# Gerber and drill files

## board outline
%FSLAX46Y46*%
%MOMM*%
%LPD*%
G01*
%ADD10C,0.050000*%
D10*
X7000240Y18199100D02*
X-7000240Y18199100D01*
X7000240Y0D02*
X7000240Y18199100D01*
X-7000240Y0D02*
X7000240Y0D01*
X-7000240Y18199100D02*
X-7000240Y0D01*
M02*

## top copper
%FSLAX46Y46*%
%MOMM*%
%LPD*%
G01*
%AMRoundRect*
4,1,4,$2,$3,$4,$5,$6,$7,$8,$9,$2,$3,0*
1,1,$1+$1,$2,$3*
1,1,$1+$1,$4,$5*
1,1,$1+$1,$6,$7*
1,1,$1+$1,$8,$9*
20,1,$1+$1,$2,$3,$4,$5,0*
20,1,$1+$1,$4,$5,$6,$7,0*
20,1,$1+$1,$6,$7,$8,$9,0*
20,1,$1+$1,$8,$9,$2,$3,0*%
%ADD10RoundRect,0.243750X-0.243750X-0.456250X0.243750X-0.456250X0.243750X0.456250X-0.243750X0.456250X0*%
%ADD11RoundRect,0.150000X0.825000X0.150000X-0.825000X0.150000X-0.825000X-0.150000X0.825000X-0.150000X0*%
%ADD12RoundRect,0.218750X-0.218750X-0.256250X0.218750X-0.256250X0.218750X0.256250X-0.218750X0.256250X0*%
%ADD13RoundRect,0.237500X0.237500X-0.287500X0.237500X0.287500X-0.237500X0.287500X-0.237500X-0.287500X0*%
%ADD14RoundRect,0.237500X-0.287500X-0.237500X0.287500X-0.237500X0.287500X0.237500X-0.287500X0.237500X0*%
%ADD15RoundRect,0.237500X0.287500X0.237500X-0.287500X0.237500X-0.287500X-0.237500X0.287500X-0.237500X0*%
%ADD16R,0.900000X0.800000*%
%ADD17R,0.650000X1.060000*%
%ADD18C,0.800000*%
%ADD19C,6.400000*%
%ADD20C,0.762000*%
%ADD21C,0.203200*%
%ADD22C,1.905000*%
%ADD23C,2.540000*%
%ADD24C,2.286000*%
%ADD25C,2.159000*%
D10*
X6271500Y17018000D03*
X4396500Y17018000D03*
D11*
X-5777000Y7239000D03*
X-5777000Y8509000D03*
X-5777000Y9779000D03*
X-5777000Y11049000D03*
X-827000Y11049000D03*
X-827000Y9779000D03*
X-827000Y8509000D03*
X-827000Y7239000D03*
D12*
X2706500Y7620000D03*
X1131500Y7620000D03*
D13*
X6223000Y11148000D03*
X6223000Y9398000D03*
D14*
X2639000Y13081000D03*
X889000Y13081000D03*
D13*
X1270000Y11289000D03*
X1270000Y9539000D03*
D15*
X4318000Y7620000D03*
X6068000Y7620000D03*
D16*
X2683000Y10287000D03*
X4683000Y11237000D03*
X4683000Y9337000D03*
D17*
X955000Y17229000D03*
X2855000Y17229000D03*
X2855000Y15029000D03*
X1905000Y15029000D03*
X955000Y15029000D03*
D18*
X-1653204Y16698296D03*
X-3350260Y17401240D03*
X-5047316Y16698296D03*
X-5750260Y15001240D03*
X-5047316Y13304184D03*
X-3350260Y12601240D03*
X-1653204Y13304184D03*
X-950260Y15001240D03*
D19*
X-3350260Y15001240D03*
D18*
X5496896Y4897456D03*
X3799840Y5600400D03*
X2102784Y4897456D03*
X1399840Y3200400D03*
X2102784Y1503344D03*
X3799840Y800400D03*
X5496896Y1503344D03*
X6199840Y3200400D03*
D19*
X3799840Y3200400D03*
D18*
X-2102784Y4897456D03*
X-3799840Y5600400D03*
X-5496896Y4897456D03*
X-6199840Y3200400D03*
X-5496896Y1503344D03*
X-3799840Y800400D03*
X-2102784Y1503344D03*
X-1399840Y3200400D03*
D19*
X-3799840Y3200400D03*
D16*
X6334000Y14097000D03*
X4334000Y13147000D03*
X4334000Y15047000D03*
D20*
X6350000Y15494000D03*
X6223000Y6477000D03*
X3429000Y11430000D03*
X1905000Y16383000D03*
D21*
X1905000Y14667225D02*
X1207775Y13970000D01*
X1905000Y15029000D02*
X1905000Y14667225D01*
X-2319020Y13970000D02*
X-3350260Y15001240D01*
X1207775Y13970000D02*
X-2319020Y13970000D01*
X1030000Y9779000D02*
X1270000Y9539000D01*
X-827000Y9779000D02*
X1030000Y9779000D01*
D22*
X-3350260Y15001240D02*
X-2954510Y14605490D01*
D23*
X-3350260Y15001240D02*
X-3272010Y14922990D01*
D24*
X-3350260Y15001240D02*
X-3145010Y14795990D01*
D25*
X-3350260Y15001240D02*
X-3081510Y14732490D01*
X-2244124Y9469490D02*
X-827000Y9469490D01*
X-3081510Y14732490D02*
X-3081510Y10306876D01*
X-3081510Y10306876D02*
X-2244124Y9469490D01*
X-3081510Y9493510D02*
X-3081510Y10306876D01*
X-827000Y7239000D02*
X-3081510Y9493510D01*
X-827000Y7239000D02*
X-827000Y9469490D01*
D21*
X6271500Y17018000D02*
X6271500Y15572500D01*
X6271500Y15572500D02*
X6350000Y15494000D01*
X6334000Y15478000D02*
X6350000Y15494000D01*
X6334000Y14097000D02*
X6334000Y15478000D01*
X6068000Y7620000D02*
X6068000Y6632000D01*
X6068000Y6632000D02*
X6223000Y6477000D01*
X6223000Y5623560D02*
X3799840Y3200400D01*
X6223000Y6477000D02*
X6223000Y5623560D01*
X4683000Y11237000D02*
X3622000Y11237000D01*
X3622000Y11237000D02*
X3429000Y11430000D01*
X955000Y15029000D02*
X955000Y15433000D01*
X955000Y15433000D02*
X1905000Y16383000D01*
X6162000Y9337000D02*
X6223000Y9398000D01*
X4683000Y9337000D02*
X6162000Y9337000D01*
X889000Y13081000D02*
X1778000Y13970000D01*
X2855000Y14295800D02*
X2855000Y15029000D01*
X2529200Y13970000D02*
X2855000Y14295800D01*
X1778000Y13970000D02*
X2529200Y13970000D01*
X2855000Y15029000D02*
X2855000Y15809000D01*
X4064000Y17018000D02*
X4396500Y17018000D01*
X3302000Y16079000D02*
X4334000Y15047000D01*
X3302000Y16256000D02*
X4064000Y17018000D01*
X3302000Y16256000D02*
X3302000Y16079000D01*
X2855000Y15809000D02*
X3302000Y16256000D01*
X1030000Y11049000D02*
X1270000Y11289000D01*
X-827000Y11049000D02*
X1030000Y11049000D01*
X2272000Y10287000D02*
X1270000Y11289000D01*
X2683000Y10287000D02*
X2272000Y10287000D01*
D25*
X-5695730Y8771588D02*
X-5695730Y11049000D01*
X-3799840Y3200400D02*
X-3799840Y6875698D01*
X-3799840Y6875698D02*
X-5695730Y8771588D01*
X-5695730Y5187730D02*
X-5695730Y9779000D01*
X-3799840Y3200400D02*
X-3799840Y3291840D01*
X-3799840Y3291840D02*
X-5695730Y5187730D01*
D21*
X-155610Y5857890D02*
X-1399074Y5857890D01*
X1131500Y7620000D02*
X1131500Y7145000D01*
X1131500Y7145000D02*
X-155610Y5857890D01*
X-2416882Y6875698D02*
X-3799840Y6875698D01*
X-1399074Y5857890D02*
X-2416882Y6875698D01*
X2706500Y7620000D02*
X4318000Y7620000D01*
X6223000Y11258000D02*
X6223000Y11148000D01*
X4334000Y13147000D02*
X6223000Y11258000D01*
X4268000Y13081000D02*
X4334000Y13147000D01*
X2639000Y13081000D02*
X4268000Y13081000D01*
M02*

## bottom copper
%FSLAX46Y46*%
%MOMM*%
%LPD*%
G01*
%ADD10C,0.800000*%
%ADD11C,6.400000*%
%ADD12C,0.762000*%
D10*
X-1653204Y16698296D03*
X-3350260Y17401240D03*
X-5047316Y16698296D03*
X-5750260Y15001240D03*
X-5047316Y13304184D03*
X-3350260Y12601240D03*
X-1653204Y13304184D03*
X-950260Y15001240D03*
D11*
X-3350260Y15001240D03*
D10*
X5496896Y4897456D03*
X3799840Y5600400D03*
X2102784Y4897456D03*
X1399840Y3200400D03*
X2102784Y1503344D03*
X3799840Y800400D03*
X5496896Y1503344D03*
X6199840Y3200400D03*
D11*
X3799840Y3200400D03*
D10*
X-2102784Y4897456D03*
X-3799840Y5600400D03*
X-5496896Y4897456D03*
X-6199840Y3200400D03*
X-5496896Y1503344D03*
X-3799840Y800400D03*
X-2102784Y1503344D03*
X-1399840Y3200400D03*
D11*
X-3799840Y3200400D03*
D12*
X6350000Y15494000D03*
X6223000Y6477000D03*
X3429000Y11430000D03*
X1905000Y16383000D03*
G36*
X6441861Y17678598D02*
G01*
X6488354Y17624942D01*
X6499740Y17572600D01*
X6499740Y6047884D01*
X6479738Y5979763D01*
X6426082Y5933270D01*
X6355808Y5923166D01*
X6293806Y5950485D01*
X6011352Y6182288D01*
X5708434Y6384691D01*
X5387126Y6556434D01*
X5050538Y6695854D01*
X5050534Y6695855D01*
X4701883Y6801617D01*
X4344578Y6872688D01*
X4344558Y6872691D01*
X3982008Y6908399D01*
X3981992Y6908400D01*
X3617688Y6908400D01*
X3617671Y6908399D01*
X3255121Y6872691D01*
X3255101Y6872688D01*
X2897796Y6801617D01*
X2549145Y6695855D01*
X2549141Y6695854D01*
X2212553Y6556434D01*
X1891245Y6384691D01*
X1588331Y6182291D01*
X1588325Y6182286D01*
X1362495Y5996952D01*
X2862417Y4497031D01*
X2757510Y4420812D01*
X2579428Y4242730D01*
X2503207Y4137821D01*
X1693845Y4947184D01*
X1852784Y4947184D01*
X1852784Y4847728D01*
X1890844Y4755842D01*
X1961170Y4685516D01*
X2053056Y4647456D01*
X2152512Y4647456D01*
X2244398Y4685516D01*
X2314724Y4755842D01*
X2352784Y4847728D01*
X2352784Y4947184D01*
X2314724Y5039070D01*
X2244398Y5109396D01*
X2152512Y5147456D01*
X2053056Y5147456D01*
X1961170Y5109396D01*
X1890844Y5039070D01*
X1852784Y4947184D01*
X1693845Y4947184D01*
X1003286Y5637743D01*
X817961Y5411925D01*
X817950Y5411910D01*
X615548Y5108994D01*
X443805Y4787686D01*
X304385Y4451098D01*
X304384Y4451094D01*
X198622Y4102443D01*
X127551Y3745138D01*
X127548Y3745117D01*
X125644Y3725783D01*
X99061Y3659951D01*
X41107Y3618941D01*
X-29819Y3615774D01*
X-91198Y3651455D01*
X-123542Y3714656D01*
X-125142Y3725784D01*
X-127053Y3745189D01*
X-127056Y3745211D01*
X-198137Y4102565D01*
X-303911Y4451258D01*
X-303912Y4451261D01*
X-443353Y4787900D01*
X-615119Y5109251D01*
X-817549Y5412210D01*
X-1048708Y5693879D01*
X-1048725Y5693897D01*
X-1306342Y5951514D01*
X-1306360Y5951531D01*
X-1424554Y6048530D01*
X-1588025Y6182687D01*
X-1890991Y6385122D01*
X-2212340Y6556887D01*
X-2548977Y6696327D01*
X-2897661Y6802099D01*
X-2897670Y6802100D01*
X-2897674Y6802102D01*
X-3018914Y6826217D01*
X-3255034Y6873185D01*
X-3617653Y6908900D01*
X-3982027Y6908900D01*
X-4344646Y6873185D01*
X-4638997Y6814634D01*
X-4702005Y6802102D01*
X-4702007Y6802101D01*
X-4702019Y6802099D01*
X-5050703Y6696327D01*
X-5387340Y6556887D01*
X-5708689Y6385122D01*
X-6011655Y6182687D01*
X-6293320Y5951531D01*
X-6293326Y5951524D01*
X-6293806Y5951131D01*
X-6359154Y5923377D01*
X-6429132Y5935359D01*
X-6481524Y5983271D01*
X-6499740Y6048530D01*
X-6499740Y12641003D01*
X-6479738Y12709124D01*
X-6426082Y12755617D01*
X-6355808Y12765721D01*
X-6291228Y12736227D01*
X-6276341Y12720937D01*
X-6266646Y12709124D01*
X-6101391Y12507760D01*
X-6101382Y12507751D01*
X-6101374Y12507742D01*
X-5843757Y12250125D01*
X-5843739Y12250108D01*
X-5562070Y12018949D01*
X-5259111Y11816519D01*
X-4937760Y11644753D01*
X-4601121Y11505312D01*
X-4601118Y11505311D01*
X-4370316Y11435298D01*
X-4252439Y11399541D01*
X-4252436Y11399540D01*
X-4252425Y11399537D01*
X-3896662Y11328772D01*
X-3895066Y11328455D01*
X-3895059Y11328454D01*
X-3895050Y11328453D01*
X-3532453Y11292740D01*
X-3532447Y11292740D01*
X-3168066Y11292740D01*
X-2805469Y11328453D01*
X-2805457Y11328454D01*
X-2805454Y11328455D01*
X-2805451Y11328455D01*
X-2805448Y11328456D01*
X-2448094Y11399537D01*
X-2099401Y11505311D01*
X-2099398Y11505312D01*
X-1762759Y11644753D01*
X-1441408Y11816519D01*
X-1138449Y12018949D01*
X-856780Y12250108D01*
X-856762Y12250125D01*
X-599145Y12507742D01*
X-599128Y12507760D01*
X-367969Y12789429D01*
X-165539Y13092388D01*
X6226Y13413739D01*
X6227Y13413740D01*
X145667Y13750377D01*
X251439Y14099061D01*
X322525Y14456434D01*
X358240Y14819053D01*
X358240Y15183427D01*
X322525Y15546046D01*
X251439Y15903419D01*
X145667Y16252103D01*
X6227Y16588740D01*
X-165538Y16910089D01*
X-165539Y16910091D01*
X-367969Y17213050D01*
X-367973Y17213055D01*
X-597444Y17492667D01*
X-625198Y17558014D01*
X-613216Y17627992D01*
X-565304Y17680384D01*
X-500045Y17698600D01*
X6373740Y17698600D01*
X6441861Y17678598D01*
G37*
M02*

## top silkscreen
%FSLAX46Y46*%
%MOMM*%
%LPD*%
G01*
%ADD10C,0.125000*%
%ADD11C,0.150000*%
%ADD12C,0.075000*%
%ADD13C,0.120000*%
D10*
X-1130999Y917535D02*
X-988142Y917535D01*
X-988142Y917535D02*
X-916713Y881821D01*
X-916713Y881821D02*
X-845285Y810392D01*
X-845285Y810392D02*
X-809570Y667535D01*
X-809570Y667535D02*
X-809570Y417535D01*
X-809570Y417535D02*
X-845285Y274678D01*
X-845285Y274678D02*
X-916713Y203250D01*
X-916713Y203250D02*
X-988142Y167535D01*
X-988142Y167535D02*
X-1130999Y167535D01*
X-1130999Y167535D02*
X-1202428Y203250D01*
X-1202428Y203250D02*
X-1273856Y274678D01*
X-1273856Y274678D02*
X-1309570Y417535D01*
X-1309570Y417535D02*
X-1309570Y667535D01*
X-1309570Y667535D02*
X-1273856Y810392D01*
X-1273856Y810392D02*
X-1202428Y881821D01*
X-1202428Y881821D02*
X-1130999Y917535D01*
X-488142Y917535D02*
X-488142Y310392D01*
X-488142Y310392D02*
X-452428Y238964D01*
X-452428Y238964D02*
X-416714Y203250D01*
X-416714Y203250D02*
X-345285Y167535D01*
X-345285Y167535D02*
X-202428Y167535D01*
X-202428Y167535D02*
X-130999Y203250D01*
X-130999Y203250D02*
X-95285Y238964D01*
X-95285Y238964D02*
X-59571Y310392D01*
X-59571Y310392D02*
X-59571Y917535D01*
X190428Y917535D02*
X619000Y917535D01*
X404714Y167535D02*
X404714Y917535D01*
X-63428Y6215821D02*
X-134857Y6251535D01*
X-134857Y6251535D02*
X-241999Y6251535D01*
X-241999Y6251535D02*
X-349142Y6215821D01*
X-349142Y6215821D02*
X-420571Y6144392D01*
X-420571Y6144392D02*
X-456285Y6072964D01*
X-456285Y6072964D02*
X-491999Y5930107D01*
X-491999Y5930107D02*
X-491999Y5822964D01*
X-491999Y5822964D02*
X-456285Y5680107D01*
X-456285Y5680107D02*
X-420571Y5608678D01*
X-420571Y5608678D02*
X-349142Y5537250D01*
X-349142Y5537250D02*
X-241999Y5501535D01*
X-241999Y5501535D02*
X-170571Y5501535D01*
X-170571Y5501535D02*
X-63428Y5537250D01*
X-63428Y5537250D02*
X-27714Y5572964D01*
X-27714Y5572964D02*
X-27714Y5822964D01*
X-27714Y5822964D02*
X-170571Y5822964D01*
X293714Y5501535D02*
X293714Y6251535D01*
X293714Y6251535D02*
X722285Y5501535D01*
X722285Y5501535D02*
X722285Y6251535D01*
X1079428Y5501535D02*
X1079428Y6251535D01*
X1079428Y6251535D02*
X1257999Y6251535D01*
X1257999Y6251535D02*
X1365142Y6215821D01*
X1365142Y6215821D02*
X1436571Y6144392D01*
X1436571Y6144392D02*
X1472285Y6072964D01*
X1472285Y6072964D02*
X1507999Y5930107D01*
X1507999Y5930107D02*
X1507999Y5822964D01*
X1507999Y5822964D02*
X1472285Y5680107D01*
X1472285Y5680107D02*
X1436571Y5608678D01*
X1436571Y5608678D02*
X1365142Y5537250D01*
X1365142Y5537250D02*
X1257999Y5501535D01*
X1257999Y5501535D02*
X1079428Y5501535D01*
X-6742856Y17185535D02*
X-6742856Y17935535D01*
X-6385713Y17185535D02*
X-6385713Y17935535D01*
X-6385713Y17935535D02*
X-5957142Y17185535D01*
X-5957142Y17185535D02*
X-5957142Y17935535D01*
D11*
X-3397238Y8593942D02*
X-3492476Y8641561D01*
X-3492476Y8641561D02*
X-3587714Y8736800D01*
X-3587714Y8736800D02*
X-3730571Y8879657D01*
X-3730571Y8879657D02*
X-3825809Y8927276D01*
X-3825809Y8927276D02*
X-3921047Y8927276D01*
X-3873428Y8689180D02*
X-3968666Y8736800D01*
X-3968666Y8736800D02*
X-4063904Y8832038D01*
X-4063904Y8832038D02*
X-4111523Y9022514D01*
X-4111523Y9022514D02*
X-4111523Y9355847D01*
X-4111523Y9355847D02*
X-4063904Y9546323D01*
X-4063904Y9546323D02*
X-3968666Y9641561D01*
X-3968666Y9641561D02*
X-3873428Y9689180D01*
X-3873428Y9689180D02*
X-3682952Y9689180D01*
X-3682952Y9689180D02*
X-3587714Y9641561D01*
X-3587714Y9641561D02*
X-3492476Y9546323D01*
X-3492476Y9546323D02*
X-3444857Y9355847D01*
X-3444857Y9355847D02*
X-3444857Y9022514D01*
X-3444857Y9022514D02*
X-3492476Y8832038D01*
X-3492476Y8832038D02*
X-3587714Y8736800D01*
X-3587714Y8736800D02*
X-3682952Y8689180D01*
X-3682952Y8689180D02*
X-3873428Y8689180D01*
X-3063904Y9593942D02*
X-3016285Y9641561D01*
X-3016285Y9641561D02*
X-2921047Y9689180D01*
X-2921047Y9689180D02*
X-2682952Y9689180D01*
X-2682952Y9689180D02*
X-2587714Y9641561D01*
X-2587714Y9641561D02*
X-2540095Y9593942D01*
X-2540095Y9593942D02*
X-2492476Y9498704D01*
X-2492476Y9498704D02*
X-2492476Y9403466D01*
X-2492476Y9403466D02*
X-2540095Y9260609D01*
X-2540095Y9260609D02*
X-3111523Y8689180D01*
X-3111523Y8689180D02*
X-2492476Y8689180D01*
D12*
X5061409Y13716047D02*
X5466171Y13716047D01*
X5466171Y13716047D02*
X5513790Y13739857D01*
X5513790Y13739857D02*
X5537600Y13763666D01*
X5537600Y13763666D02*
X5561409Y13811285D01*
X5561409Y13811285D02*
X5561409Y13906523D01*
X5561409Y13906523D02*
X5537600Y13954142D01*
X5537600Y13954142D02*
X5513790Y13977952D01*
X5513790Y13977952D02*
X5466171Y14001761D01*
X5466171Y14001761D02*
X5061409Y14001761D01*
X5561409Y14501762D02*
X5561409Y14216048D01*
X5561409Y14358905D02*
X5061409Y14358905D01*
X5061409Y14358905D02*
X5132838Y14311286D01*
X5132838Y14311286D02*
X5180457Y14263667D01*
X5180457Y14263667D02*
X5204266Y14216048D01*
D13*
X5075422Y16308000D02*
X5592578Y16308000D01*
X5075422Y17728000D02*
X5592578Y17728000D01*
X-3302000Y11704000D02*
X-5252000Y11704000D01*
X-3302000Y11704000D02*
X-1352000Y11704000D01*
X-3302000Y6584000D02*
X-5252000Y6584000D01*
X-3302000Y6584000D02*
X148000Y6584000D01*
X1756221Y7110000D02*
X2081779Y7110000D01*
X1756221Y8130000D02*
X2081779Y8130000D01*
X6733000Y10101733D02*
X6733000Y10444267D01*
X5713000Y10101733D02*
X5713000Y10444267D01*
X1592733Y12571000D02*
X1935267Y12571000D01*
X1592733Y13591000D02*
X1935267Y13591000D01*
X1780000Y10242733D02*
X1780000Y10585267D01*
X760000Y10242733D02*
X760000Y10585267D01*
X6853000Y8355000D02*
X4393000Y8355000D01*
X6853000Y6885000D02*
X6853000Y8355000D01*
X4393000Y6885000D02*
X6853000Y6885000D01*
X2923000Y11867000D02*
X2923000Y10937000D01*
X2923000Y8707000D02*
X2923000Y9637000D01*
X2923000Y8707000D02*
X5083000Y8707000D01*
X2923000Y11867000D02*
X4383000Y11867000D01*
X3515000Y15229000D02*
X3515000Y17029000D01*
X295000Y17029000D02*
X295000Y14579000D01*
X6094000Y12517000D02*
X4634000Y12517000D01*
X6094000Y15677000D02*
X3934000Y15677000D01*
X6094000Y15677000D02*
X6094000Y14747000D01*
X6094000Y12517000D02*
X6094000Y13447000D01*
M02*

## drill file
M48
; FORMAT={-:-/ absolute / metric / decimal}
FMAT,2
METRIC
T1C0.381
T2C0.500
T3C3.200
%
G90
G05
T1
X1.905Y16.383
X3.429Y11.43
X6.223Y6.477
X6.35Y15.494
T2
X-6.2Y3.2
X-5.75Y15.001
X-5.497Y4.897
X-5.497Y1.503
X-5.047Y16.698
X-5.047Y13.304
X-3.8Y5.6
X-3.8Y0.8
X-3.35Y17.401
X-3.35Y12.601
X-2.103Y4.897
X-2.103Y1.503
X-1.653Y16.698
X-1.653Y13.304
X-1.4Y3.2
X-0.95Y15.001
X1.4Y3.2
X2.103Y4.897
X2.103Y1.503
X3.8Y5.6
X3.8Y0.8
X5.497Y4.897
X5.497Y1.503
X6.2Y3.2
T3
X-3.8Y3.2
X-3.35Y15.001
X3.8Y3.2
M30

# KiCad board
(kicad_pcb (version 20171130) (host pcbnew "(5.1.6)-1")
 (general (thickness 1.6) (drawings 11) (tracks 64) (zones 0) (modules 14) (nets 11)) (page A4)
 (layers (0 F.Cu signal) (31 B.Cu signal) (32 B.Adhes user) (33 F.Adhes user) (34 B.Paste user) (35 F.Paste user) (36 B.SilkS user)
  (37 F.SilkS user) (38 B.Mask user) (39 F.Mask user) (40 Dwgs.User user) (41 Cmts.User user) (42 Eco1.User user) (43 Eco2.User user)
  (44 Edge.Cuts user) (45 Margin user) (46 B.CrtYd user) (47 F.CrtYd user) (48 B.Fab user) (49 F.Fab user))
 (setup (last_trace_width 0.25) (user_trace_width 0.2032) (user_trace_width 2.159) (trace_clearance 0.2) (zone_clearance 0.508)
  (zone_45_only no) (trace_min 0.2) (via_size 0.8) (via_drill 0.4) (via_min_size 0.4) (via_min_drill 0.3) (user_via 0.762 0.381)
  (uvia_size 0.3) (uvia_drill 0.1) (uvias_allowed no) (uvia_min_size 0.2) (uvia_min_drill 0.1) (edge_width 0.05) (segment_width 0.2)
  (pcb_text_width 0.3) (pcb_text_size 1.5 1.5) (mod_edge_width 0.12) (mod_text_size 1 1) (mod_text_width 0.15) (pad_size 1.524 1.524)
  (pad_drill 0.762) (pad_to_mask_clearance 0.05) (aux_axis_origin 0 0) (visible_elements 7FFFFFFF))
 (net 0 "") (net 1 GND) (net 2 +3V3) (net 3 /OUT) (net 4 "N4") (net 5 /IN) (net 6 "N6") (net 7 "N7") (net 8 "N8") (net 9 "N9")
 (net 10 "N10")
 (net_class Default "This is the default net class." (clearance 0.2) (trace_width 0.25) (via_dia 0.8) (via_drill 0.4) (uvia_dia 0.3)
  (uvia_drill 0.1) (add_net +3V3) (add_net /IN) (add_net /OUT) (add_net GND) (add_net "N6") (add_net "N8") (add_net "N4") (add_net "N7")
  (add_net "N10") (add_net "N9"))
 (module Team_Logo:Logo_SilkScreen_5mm (layer B.Cu) (at 3.429 -15.621 180)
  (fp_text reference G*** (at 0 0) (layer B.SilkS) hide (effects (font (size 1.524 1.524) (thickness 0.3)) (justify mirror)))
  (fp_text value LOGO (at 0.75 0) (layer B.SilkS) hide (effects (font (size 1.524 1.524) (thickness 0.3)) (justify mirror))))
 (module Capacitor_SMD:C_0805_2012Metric (layer F.Cu) (at 5.334 -17.018)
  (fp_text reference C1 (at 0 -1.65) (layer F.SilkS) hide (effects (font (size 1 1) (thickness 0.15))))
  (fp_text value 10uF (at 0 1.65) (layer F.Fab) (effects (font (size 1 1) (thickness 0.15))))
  (fp_line (start -0.258578 0.71) (end 0.258578 0.71) (layer F.SilkS) (width 0.12))
  (fp_line (start -0.258578 -0.71) (end 0.258578 -0.71) (layer F.SilkS) (width 0.12))
  (pad 2 smd roundrect (at 0.9375 0) (size 0.975 1.4) (layers F.Cu F.Paste F.Mask) (roundrect_rratio 0.25) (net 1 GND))
  (pad 1 smd roundrect (at -0.9375 0) (size 0.975 1.4) (layers F.Cu F.Paste F.Mask) (roundrect_rratio 0.25) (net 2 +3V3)))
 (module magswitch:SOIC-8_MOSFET (layer F.Cu) (at -3.302 -9.144 180)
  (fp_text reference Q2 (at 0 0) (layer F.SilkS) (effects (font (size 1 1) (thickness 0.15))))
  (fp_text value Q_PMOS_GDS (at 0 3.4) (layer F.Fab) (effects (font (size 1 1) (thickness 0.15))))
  (fp_line (start 0 2.56) (end 1.95 2.56) (layer F.SilkS) (width 0.12))
  (fp_line (start 0 2.56) (end -1.95 2.56) (layer F.SilkS) (width 0.12))
  (fp_line (start 0 -2.56) (end 1.95 -2.56) (layer F.SilkS) (width 0.12))
  (fp_line (start 0 -2.56) (end -3.45 -2.56) (layer F.SilkS) (width 0.12))
  (pad 2 smd roundrect (at 2.475 -1.905 180) (size 1.95 0.6) (layers F.Cu F.Paste F.Mask) (roundrect_rratio 0.25) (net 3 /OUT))
  (pad 2 smd roundrect (at 2.475 -0.635 180) (size 1.95 0.6) (layers F.Cu F.Paste F.Mask) (roundrect_rratio 0.25) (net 3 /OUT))
  (pad 2 smd roundrect (at 2.475 0.635 180) (size 1.95 0.6) (layers F.Cu F.Paste F.Mask) (roundrect_rratio 0.25) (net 3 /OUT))
  (pad 2 smd roundrect (at 2.475 1.905 180) (size 1.95 0.6) (layers F.Cu F.Paste F.Mask) (roundrect_rratio 0.25) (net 3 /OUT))
  (pad 1 smd roundrect (at -2.475 1.905 180) (size 1.95 0.6) (layers F.Cu F.Paste F.Mask) (roundrect_rratio 0.25) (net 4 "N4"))
  (pad 3 smd roundrect (at -2.475 0.635 180) (size 1.95 0.6) (layers F.Cu F.Paste F.Mask) (roundrect_rratio 0.25) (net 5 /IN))
  (pad 3 smd roundrect (at -2.475 -0.635 180) (size 1.95 0.6) (layers F.Cu F.Paste F.Mask) (roundrect_rratio 0.25) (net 5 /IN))
  (pad 3 smd roundrect (at -2.475 -1.905 180) (size 1.95 0.6) (layers F.Cu F.Paste F.Mask) (roundrect_rratio 0.25) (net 5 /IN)))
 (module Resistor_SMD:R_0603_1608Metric (layer F.Cu) (at 1.919 -7.62)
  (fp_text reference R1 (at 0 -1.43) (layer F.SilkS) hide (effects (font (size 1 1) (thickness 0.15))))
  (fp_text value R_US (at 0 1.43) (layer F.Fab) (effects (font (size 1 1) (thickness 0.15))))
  (fp_line (start -0.162779 0.51) (end 0.162779 0.51) (layer F.SilkS) (width 0.12))
  (fp_line (start -0.162779 -0.51) (end 0.162779 -0.51) (layer F.SilkS) (width 0.12))
  (pad 2 smd roundrect (at 0.7875 0) (size 0.875 0.95) (layers F.Cu F.Paste F.Mask) (roundrect_rratio 0.25) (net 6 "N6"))
  (pad 1 smd roundrect (at -0.7875 0) (size 0.875 0.95) (layers F.Cu F.Paste F.Mask) (roundrect_rratio 0.25) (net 3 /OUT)))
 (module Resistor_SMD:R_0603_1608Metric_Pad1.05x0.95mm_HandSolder (layer F.Cu) (at 6.223 -10.273 90)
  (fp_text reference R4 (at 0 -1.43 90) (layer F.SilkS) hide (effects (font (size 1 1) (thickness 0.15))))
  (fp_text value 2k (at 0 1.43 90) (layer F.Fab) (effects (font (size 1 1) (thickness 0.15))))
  (fp_line (start -0.171267 0.51) (end 0.171267 0.51) (layer F.SilkS) (width 0.12))
  (fp_line (start -0.171267 -0.51) (end 0.171267 -0.51) (layer F.SilkS) (width 0.12))
  (pad 2 smd roundrect (at 0.875 0 90) (size 1.05 0.95) (layers F.Cu F.Paste F.Mask) (roundrect_rratio 0.25) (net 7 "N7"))
  (pad 1 smd roundrect (at -0.875 0 90) (size 1.05 0.95) (layers F.Cu F.Paste F.Mask) (roundrect_rratio 0.25) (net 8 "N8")))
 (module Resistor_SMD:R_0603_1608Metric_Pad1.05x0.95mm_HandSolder (layer F.Cu) (at 1.764 -13.081)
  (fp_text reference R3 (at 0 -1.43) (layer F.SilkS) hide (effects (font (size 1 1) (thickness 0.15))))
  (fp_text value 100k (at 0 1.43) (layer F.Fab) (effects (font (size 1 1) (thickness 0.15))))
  (fp_line (start -0.171267 0.51) (end 0.171267 0.51) (layer F.SilkS) (width 0.12))
  (fp_line (start -0.171267 -0.51) (end 0.171267 -0.51) (layer F.SilkS) (width 0.12))
  (pad 2 smd roundrect (at 0.875 0) (size 1.05 0.95) (layers F.Cu F.Paste F.Mask) (roundrect_rratio 0.25) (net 7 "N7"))
  (pad 1 smd roundrect (at -0.875 0) (size 1.05 0.95) (layers F.Cu F.Paste F.Mask) (roundrect_rratio 0.25) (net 2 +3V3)))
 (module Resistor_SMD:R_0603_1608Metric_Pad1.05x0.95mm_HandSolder (layer F.Cu) (at 1.27 -10.414 90)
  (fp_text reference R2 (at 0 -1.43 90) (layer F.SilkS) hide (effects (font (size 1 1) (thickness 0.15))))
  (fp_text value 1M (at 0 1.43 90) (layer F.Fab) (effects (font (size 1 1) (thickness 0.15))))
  (fp_line (start -0.171267 0.51) (end 0.171267 0.51) (layer F.SilkS) (width 0.12))
  (fp_line (start -0.171267 -0.51) (end 0.171267 -0.51) (layer F.SilkS) (width 0.12))
  (pad 2 smd roundrect (at 0.875 0 90) (size 1.05 0.95) (layers F.Cu F.Paste F.Mask) (roundrect_rratio 0.25) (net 4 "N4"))
  (pad 1 smd roundrect (at -0.875 0 90) (size 1.05 0.95) (layers F.Cu F.Paste F.Mask) (roundrect_rratio 0.25) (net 5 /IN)))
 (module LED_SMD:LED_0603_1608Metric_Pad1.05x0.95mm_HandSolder (layer F.Cu) (at 5.193 -7.62 180)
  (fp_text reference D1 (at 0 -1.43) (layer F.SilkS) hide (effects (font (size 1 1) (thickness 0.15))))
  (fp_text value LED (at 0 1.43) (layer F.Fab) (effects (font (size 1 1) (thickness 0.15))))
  (fp_line (start -1.66 0.735) (end 0.8 0.735) (layer F.SilkS) (width 0.12))
  (fp_line (start -1.66 -0.735) (end -1.66 0.735) (layer F.SilkS) (width 0.12))
  (fp_line (start 0.8 -0.735) (end -1.66 -0.735) (layer F.SilkS) (width 0.12))
  (pad 2 smd roundrect (at 0.875 0 180) (size 1.05 0.95) (layers F.Cu F.Paste F.Mask) (roundrect_rratio 0.25) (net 6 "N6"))
  (pad 1 smd roundrect (at -0.875 0 180) (size 1.05 0.95) (layers F.Cu F.Paste F.Mask) (roundrect_rratio 0.25) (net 1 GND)))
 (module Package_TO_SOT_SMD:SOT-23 (layer F.Cu) (at 3.683 -10.287 180)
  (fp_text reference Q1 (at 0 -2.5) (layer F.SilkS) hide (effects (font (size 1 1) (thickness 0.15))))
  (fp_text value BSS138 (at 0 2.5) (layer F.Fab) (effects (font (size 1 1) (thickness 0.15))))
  (fp_line (start 0.76 1.58) (end 0.76 0.65) (layer F.SilkS) (width 0.12))
  (fp_line (start 0.76 -1.58) (end 0.76 -0.65) (layer F.SilkS) (width 0.12))
  (fp_line (start 0.76 -1.58) (end -1.4 -1.58) (layer F.SilkS) (width 0.12))
  (fp_line (start 0.76 1.58) (end -0.7 1.58) (layer F.SilkS) (width 0.12))
  (pad 3 smd rect (at 1 0 180) (size 0.9 0.8) (layers F.Cu F.Paste F.Mask) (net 4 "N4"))
  (pad 2 smd rect (at -1 0.95 180) (size 0.9 0.8) (layers F.Cu F.Paste F.Mask) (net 1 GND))
  (pad 1 smd rect (at -1 -0.95 180) (size 0.9 0.8) (layers F.Cu F.Paste F.Mask) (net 8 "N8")))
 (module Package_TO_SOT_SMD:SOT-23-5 (layer F.Cu) (at 1.905 -16.129 90)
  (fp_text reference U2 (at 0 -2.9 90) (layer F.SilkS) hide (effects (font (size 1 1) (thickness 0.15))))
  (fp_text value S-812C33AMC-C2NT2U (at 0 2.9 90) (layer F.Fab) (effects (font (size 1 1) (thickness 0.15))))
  (fp_line (start -0.9 1.61) (end 0.9 1.61) (layer F.SilkS) (width 0.12))
  (fp_line (start 0.9 -1.61) (end -1.55 -1.61) (layer F.SilkS) (width 0.12))
  (pad 5 smd rect (at 1.1 -0.95 90) (size 1.06 0.65) (layers F.Cu F.Paste F.Mask) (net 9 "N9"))
  (pad 4 smd rect (at 1.1 0.95 90) (size 1.06 0.65) (layers F.Cu F.Paste F.Mask) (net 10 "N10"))
  (pad 3 smd rect (at -1.1 0.95 90) (size 1.06 0.65) (layers F.Cu F.Paste F.Mask) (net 2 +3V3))
  (pad 2 smd rect (at -1.1 0 90) (size 1.06 0.65) (layers F.Cu F.Paste F.Mask) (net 5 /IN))
  (pad 1 smd rect (at -1.1 -0.95 90) (size 1.06 0.65) (layers F.Cu F.Paste F.Mask) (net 1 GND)))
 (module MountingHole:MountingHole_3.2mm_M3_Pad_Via (layer F.Cu) (at -3.35026 -15.00124)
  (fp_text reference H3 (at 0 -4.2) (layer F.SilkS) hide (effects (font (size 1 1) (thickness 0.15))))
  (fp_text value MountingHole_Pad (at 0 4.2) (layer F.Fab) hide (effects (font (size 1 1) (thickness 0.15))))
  (pad 1 thru_hole circle (at 1.697056 -1.697056) (size 0.8 0.8) (drill 0.5) (layers *.Cu *.Mask) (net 5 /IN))
  (pad 1 thru_hole circle (at 0 -2.4) (size 0.8 0.8) (drill 0.5) (layers *.Cu *.Mask) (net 5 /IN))
  (pad 1 thru_hole circle (at -1.697056 -1.697056) (size 0.8 0.8) (drill 0.5) (layers *.Cu *.Mask) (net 5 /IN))
  (pad 1 thru_hole circle (at -2.4 0) (size 0.8 0.8) (drill 0.5) (layers *.Cu *.Mask) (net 5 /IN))
  (pad 1 thru_hole circle (at -1.697056 1.697056) (size 0.8 0.8) (drill 0.5) (layers *.Cu *.Mask) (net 5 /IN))
  (pad 1 thru_hole circle (at 0 2.4) (size 0.8 0.8) (drill 0.5) (layers *.Cu *.Mask) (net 5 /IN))
  (pad 1 thru_hole circle (at 1.697056 1.697056) (size 0.8 0.8) (drill 0.5) (layers *.Cu *.Mask) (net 5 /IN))
  (pad 1 thru_hole circle (at 2.4 0) (size 0.8 0.8) (drill 0.5) (layers *.Cu *.Mask) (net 5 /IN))
  (pad 1 thru_hole circle (at 0 0) (size 6.4 6.4) (drill 3.2) (layers *.Cu *.Mask) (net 5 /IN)))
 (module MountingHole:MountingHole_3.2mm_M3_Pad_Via (layer F.Cu) (at 3.79984 -3.2004)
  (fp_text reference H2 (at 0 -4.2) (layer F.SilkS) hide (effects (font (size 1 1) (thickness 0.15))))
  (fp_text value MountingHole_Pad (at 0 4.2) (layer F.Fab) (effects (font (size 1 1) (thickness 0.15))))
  (pad 1 thru_hole circle (at 1.697056 -1.697056) (size 0.8 0.8) (drill 0.5) (layers *.Cu *.Mask) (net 1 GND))
  (pad 1 thru_hole circle (at 0 -2.4) (size 0.8 0.8) (drill 0.5) (layers *.Cu *.Mask) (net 1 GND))
  (pad 1 thru_hole circle (at -1.697056 -1.697056) (size 0.8 0.8) (drill 0.5) (layers *.Cu *.Mask) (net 1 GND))
  (pad 1 thru_hole circle (at -2.4 0) (size 0.8 0.8) (drill 0.5) (layers *.Cu *.Mask) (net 1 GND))
  (pad 1 thru_hole circle (at -1.697056 1.697056) (size 0.8 0.8) (drill 0.5) (layers *.Cu *.Mask) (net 1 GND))
  (pad 1 thru_hole circle (at 0 2.4) (size 0.8 0.8) (drill 0.5) (layers *.Cu *.Mask) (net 1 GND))
  (pad 1 thru_hole circle (at 1.697056 1.697056) (size 0.8 0.8) (drill 0.5) (layers *.Cu *.Mask) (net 1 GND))
  (pad 1 thru_hole circle (at 2.4 0) (size 0.8 0.8) (drill 0.5) (layers *.Cu *.Mask) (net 1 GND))
  (pad 1 thru_hole circle (at 0 0) (size 6.4 6.4) (drill 3.2) (layers *.Cu *.Mask) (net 1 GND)))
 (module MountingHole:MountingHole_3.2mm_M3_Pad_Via (layer F.Cu) (at -3.79984 -3.2004)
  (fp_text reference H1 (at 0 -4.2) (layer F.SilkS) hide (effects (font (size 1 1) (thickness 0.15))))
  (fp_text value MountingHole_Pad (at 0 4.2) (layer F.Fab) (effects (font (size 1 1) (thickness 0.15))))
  (pad 1 thru_hole circle (at 1.697056 -1.697056) (size 0.8 0.8) (drill 0.5) (layers *.Cu *.Mask) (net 3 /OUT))
  (pad 1 thru_hole circle (at 0 -2.4) (size 0.8 0.8) (drill 0.5) (layers *.Cu *.Mask) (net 3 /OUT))
  (pad 1 thru_hole circle (at -1.697056 -1.697056) (size 0.8 0.8) (drill 0.5) (layers *.Cu *.Mask) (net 3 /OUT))
  (pad 1 thru_hole circle (at -2.4 0) (size 0.8 0.8) (drill 0.5) (layers *.Cu *.Mask) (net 3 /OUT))
  (pad 1 thru_hole circle (at -1.697056 1.697056) (size 0.8 0.8) (drill 0.5) (layers *.Cu *.Mask) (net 3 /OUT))
  (pad 1 thru_hole circle (at 0 2.4) (size 0.8 0.8) (drill 0.5) (layers *.Cu *.Mask) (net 3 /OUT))
  (pad 1 thru_hole circle (at 1.697056 1.697056) (size 0.8 0.8) (drill 0.5) (layers *.Cu *.Mask) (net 3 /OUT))
  (pad 1 thru_hole circle (at 2.4 0) (size 0.8 0.8) (drill 0.5) (layers *.Cu *.Mask) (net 3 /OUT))
  (pad 1 thru_hole circle (at 0 0) (size 6.4 6.4) (drill 3.2) (layers *.Cu *.Mask) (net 3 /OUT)))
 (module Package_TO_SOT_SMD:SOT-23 (layer F.Cu) (at 5.334 -14.097)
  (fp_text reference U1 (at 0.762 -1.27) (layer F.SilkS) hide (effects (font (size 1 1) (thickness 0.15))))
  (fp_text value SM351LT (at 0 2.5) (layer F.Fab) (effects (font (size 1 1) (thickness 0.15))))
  (fp_line (start 0.76 1.58) (end -0.7 1.58) (layer F.SilkS) (width 0.12))
  (fp_line (start 0.76 -1.58) (end -1.4 -1.58) (layer F.SilkS) (width 0.12))
  (fp_line (start 0.76 -1.58) (end 0.76 -0.65) (layer F.SilkS) (width 0.12))
  (fp_line (start 0.76 1.58) (end 0.76 0.65) (layer F.SilkS) (width 0.12))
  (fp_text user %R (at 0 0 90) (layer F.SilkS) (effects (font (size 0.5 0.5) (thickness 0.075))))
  (pad 3 smd rect (at 1 0) (size 0.9 0.8) (layers F.Cu F.Paste F.Mask) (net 1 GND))
  (pad 2 smd rect (at -1 0.95) (size 0.9 0.8) (layers F.Cu F.Paste F.Mask) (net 7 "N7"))
  (pad 1 smd rect (at -1 -0.95) (size 0.9 0.8) (layers F.Cu F.Paste F.Mask) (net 2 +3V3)))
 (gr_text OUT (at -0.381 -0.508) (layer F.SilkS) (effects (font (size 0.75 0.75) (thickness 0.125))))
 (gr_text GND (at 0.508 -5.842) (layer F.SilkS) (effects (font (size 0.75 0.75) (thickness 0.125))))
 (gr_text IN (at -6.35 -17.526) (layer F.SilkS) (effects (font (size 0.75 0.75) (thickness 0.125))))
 (gr_line (start 7.00024 -18.1991) (end -7.00024 -18.1991) (layer Edge.Cuts) (width 0.05))
 (gr_line (start 7.00024 0) (end 7.00024 -18.1991) (layer Edge.Cuts) (width 0.05))
 (gr_line (start -7.00024 0) (end 7.00024 0) (layer Edge.Cuts) (width 0.05))
 (gr_line (start -7.00024 -18.1991) (end -7.00024 0) (layer Edge.Cuts) (width 0.05))
 (segment (start 1.905 -14.667225) (end 1.207775 -13.97) (width 0.2032) (layer F.Cu) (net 5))
 (segment (start 1.905 -15.029) (end 1.905 -14.667225) (width 0.2032) (layer F.Cu) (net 5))
 (segment (start -2.31902 -13.97) (end -3.35026 -15.00124) (width 0.2032) (layer F.Cu) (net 5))
 (segment (start 1.207775 -13.97) (end -2.31902 -13.97) (width 0.2032) (layer F.Cu) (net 5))
 (segment (start 1.03 -9.779) (end 1.27 -9.539) (width 0.2032) (layer F.Cu) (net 5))
 (segment (start -0.827 -9.779) (end 1.03 -9.779) (width 0.2032) (layer F.Cu) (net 5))
 (segment (start -3.35026 -15.00124) (end -2.95451 -14.60549) (width 1.905) (layer F.Cu) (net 5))
 (segment (start -3.35026 -15.00124) (end -3.27201 -14.92299) (width 2.54) (layer F.Cu) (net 5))
 (segment (start -3.35026 -15.00124) (end -3.14501 -14.79599) (width 2.286) (layer F.Cu) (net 5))
 (segment (start -3.35026 -15.00124) (end -3.08151 -14.73249) (width 2.159) (layer F.Cu) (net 5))
 (segment (start -2.244124 -9.46949) (end -0.827 -9.46949) (width 2.159) (layer F.Cu) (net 5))
 (segment (start -3.08151 -14.73249) (end -3.08151 -10.306876) (width 2.159) (layer F.Cu) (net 5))
 (segment (start -3.08151 -10.306876) (end -2.244124 -9.46949) (width 2.159) (layer F.Cu) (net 5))
 (segment (start -3.08151 -9.49351) (end -3.08151 -10.306876) (width 2.159) (layer F.Cu) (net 5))
 (segment (start -0.827 -7.239) (end -3.08151 -9.49351) (width 2.159) (layer F.Cu) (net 5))
 (segment (start -0.827 -7.239) (end -0.827 -9.46949) (width 2.159) (layer F.Cu) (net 5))
 (via (at 6.35 -15.494) (size 0.762) (drill 0.381) (layers F.Cu B.Cu) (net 1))
 (segment (start 6.2715 -17.018) (end 6.2715 -15.5725) (width 0.2032) (layer F.Cu) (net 1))
 (segment (start 6.2715 -15.5725) (end 6.35 -15.494) (width 0.2032) (layer F.Cu) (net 1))
 (segment (start 6.334 -15.478) (end 6.35 -15.494) (width 0.2032) (layer F.Cu) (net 1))
 (segment (start 6.334 -14.097) (end 6.334 -15.478) (width 0.2032) (layer F.Cu) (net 1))
 (via (at 6.223 -6.477) (size 0.762) (drill 0.381) (layers F.Cu B.Cu) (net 1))
 (segment (start 6.068 -7.62) (end 6.068 -6.632) (width 0.2032) (layer F.Cu) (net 1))
 (segment (start 6.068 -6.632) (end 6.223 -6.477) (width 0.2032) (layer F.Cu) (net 1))
 (segment (start 6.223 -5.62356) (end 3.79984 -3.2004) (width 0.2032) (layer F.Cu) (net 1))
 (segment (start 6.223 -6.477) (end 6.223 -5.62356) (width 0.2032) (layer F.Cu) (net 1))
 (segment (start 4.683 -11.237) (end 3.622 -11.237) (width 0.2032) (layer F.Cu) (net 1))
 (via (at 3.429 -11.43) (size 0.762) (drill 0.381) (layers F.Cu B.Cu) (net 1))
 (segment (start 3.622 -11.237) (end 3.429 -11.43) (width 0.2032) (layer F.Cu) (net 1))
 (segment (start 0.955 -15.029) (end 0.955 -15.433) (width 0.2032) (layer F.Cu) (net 1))
 (via (at 1.905 -16.383) (size 0.762) (drill 0.381) (layers F.Cu B.Cu) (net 1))
 (segment (start 0.955 -15.433) (end 1.905 -16.383) (width 0.2032) (layer F.Cu) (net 1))
 (segment (start 6.162 -9.337) (end 6.223 -9.398) (width 0.2032) (layer F.Cu) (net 8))
 (segment (start 4.683 -9.337) (end 6.162 -9.337) (width 0.2032) (layer F.Cu) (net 8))
 (segment (start 0.889 -13.081) (end 1.778 -13.97) (width 0.2032) (layer F.Cu) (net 2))
 (segment (start 2.855 -14.2958) (end 2.855 -15.029) (width 0.2032) (layer F.Cu) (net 2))
 (segment (start 2.5292 -13.97) (end 2.855 -14.2958) (width 0.2032) (layer F.Cu) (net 2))
 (segment (start 1.778 -13.97) (end 2.5292 -13.97) (width 0.2032) (layer F.Cu) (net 2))
 (segment (start 2.855 -15.029) (end 2.855 -15.809) (width 0.2032) (layer F.Cu) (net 2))
 (segment (start 4.064 -17.018) (end 4.3965 -17.018) (width 0.2032) (layer F.Cu) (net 2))
 (segment (start 3.302 -16.079) (end 4.334 -15.047) (width 0.2032) (layer F.Cu) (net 2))
 (segment (start 3.302 -16.256) (end 4.064 -17.018) (width 0.2032) (layer F.Cu) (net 2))
 (segment (start 3.302 -16.256) (end 3.302 -16.079) (width 0.2032) (layer F.Cu) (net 2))
 (segment (start 2.855 -15.809) (end 3.302 -16.256) (width 0.2032) (layer F.Cu) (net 2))
 (segment (start 1.03 -11.049) (end 1.27 -11.289) (width 0.2032) (layer F.Cu) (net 4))
 (segment (start -0.827 -11.049) (end 1.03 -11.049) (width 0.2032) (layer F.Cu) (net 4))
 (segment (start 2.272 -10.287) (end 1.27 -11.289) (width 0.2032) (layer F.Cu) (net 4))
 (segment (start 2.683 -10.287) (end 2.272 -10.287) (width 0.2032) (layer F.Cu) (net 4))
 (segment (start -5.69573 -8.771588) (end -5.69573 -11.049) (width 2.159) (layer F.Cu) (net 3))
 (segment (start -3.79984 -3.2004) (end -3.79984 -6.875698) (width 2.159) (layer F.Cu) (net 3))
 (segment (start -3.79984 -6.875698) (end -5.69573 -8.771588) (width 2.159) (layer F.Cu) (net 3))
 (segment (start -5.69573 -5.18773) (end -5.69573 -9.779) (width 2.159) (layer F.Cu) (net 3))
 (segment (start -3.79984 -3.2004) (end -3.79984 -3.29184) (width 2.159) (layer F.Cu) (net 3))
 (segment (start -3.79984 -3.29184) (end -5.69573 -5.18773) (width 2.159) (layer F.Cu) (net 3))
 (segment (start -0.15561 -5.85789) (end -1.399074 -5.85789) (width 0.2032) (layer F.Cu) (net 3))
 (segment (start 1.1315 -7.62) (end 1.1315 -7.145) (width 0.2032) (layer F.Cu) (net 3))
 (segment (start 1.1315 -7.145) (end -0.15561 -5.85789) (width 0.2032) (layer F.Cu) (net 3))
 (segment (start -2.416882 -6.875698) (end -3.79984 -6.875698) (width 0.2032) (layer F.Cu) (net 3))
 (segment (start -1.399074 -5.85789) (end -2.416882 -6.875698) (width 0.2032) (layer F.Cu) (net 3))
 (segment (start 2.7065 -7.62) (end 4.318 -7.62) (width 0.2032) (layer F.Cu) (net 6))
 (segment (start 6.223 -11.258) (end 6.223 -11.148) (width 0.2032) (layer F.Cu) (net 7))
 (segment (start 4.334 -13.147) (end 6.223 -11.258) (width 0.2032) (layer F.Cu) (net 7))
 (segment (start 4.268 -13.081) (end 4.334 -13.147) (width 0.2032) (layer F.Cu) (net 7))
 (segment (start 2.639 -13.081) (end 4.268 -13.081) (width 0.2032) (layer F.Cu) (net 7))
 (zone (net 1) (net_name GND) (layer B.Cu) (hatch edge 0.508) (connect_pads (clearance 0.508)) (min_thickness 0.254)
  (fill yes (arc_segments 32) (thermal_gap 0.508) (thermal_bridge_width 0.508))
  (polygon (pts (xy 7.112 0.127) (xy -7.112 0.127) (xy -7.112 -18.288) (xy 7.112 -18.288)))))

